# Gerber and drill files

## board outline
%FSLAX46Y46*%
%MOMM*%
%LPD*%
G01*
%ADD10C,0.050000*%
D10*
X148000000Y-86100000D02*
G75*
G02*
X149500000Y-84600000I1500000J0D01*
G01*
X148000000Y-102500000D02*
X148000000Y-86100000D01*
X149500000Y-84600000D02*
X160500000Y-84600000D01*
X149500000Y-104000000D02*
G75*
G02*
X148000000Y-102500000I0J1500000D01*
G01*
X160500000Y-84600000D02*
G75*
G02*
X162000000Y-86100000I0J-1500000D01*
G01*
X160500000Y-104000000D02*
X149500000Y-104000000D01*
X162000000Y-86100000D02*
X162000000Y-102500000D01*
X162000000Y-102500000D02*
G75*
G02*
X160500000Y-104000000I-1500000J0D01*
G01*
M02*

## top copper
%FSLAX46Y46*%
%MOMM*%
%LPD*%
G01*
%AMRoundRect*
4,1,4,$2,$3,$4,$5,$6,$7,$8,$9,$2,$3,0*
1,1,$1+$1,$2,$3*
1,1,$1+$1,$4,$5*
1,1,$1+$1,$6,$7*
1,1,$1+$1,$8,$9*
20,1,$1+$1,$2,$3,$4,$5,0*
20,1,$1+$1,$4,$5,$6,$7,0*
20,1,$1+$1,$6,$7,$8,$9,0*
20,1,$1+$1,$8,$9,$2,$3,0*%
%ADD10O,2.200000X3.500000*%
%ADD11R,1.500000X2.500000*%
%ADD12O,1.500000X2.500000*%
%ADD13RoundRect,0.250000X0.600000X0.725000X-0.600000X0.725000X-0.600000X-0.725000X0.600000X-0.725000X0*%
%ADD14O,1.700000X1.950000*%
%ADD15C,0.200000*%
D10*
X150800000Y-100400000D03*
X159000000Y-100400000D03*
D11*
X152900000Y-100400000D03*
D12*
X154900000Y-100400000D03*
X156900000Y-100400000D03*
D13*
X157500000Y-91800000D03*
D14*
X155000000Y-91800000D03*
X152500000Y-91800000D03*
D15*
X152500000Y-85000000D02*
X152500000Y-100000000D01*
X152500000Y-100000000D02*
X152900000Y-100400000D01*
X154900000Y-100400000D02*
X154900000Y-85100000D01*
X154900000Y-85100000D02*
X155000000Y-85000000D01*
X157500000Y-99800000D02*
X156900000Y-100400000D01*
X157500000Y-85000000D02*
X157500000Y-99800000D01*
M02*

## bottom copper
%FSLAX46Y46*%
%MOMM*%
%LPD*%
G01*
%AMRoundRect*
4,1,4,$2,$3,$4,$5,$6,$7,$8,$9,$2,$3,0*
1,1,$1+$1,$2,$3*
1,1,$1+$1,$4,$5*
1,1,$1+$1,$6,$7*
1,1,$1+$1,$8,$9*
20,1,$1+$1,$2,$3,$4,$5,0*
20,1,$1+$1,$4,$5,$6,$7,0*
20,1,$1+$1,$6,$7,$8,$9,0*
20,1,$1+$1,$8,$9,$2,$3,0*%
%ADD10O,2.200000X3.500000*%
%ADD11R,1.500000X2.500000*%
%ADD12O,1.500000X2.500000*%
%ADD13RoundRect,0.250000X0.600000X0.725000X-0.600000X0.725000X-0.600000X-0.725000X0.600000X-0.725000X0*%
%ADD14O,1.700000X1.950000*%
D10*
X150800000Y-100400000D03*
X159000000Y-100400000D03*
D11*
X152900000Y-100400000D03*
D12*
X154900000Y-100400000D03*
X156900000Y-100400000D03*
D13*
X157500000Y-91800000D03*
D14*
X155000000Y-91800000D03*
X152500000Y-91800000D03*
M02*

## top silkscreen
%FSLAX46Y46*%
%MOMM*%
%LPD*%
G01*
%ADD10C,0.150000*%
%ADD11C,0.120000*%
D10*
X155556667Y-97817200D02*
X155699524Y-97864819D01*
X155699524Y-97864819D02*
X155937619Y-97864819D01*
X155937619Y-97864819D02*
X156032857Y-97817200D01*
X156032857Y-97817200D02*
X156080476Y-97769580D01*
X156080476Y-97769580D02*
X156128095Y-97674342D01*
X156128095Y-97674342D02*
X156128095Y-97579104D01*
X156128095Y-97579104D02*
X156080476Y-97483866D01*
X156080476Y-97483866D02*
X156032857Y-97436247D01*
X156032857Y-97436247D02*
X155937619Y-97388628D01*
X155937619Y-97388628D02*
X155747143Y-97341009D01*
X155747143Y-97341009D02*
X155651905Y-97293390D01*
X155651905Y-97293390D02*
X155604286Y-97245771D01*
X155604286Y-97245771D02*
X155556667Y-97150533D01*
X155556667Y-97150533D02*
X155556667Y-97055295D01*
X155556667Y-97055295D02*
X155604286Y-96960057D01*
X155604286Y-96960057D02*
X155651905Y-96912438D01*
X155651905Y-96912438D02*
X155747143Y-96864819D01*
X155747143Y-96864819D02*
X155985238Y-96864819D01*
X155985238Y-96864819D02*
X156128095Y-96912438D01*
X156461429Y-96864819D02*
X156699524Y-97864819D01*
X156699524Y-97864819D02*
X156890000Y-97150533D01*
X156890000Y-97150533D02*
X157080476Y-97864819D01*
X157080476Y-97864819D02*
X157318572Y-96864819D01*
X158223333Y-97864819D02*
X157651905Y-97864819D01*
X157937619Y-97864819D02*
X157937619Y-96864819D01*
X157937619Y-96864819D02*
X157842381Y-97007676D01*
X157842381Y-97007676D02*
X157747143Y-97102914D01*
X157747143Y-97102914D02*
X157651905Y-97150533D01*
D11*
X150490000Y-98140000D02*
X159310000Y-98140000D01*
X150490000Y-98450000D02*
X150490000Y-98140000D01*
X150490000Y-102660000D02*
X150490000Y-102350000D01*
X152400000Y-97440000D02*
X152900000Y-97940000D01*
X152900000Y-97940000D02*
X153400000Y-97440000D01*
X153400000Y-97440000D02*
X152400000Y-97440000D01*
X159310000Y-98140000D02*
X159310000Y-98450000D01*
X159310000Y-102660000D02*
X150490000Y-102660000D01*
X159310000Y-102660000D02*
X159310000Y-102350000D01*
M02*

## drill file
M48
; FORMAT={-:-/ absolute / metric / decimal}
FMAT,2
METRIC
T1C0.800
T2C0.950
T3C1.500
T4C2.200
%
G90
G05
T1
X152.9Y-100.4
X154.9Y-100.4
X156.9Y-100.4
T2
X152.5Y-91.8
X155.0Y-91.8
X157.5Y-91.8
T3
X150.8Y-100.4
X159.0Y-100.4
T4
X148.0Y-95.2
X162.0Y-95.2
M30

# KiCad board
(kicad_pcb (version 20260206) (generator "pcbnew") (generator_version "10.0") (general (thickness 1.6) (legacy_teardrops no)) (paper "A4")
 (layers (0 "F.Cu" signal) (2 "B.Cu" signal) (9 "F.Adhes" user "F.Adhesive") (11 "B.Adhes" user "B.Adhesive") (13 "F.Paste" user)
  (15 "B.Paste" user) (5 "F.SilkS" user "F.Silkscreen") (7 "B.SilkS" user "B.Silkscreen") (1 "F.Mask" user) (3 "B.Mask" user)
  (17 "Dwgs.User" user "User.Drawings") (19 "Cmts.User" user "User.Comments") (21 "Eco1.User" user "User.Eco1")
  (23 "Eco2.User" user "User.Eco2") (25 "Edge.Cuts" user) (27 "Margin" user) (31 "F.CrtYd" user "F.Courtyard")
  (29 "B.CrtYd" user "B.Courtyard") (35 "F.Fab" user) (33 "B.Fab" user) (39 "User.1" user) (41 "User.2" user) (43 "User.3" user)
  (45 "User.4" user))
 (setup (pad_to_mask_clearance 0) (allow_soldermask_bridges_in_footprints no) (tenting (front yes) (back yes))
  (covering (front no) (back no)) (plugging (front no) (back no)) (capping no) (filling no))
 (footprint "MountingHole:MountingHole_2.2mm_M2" (layer "F.Cu") (at 162 95.2)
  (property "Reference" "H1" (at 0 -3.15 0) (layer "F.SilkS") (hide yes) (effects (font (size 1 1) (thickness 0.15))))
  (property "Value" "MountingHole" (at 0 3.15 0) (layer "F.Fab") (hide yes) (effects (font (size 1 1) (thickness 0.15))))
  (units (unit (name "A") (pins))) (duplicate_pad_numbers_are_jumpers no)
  (pad "" np_thru_hole circle (at 0 0) (size 2.2 2.2) (drill 2.2) (layers "*.Cu" "*.Mask")))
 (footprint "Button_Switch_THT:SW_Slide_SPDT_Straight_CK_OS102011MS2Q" (layer "F.Cu") (at 152.9 100.4)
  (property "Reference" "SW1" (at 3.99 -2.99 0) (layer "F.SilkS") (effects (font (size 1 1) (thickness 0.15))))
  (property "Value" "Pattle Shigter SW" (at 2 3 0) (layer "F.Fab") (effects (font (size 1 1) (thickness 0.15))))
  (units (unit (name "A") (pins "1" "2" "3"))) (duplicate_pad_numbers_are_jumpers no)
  (fp_line (start -2.41 -2.26) (end 6.41 -2.26) (stroke (width 0.12) (type solid)) (layer "F.SilkS"))
  (fp_line (start -2.41 -1.95) (end -2.41 -2.26) (stroke (width 0.12) (type solid)) (layer "F.SilkS"))
  (fp_line (start -2.41 2.26) (end -2.41 1.95) (stroke (width 0.12) (type solid)) (layer "F.SilkS"))
  (fp_line (start -0.5 -2.96) (end 0 -2.46) (stroke (width 0.12) (type solid)) (layer "F.SilkS"))
  (fp_line (start 0 -2.46) (end 0.5 -2.96) (stroke (width 0.12) (type solid)) (layer "F.SilkS"))
  (fp_line (start 0.5 -2.96) (end -0.5 -2.96) (stroke (width 0.12) (type solid)) (layer "F.SilkS"))
  (fp_line (start 6.41 -2.26) (end 6.41 -1.95) (stroke (width 0.12) (type solid)) (layer "F.SilkS"))
  (fp_line (start 6.41 2.26) (end -2.41 2.26) (stroke (width 0.12) (type solid)) (layer "F.SilkS"))
  (fp_line (start 6.41 2.26) (end 6.41 1.95) (stroke (width 0.12) (type solid)) (layer "F.SilkS"))
  (pad "" thru_hole oval (at -2.1 0) (size 2.2 3.5) (drill 1.5) (layers "*.Cu" "*.Mask") (remove_unused_layers no))
  (pad "" thru_hole oval (at 6.1 0) (size 2.2 3.5) (drill 1.5) (layers "*.Cu" "*.Mask") (remove_unused_layers no))
  (pad "1" thru_hole rect (at 0 0) (size 1.5 2.5) (drill 0.8) (layers "*.Cu" "*.Mask") (remove_unused_layers no) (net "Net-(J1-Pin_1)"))
  (pad "2" thru_hole oval (at 2 0) (size 1.5 2.5) (drill 0.8) (layers "*.Cu" "*.Mask") (remove_unused_layers no) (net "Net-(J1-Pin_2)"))
  (pad "3" thru_hole oval (at 4 0) (size 1.5 2.5) (drill 0.8) (layers "*.Cu" "*.Mask") (remove_unused_layers no) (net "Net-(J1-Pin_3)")))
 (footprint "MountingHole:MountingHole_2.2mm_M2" (layer "F.Cu") (at 148 95.2)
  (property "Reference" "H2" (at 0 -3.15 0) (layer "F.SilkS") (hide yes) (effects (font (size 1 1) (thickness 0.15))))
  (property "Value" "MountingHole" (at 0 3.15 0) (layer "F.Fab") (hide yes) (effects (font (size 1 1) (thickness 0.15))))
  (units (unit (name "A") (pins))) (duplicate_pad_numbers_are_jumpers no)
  (pad "" np_thru_hole circle (at 0 0) (size 2.2 2.2) (drill 2.2) (layers "*.Cu" "*.Mask")))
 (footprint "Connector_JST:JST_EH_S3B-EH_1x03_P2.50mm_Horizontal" (layer "B.Cu") (at 157.5 91.8 180)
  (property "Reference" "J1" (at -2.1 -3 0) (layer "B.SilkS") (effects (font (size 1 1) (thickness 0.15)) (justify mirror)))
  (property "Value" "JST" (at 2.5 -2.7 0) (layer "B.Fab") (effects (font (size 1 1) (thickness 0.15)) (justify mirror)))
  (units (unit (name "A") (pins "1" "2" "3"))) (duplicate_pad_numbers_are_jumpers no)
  (pad "1" thru_hole roundrect (at 0 0 180) (size 1.7 1.95) (drill 0.95) (layers "*.Cu" "*.Mask") (remove_unused_layers no)
   (roundrect_rratio 0.147059) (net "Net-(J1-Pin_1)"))
  (pad "2" thru_hole oval (at 2.5 0 180) (size 1.7 1.95) (drill 0.95) (layers "*.Cu" "*.Mask") (remove_unused_layers no)
   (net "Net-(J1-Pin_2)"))
  (pad "3" thru_hole oval (at 5 0 180) (size 1.7 1.95) (drill 0.95) (layers "*.Cu" "*.Mask") (remove_unused_layers no)
   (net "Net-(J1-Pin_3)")))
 (gr_arc (start 148 86.1) (mid 148.43934 85.03934) (end 149.5 84.6) (stroke (width 0.05) (type default)) (layer "Edge.Cuts"))
 (gr_line (start 148 102.5) (end 148 86.1) (stroke (width 0.05) (type default)) (layer "Edge.Cuts"))
 (gr_line (start 149.5 84.6) (end 160.5 84.6) (stroke (width 0.05) (type default)) (layer "Edge.Cuts"))
 (gr_arc (start 149.5 104) (mid 148.43934 103.56066) (end 148 102.5) (stroke (width 0.05) (type default)) (layer "Edge.Cuts"))
 (gr_arc (start 160.5 84.6) (mid 161.56066 85.03934) (end 162 86.1) (stroke (width 0.05) (type default)) (layer "Edge.Cuts"))
 (gr_line (start 160.5 104) (end 149.5 104) (stroke (width 0.05) (type default)) (layer "Edge.Cuts"))
 (gr_line (start 162 86.1) (end 162 102.5) (stroke (width 0.05) (type default)) (layer "Edge.Cuts"))
 (gr_arc (start 162 102.5) (mid 161.56066 103.56066) (end 160.5 104) (stroke (width 0.05) (type default)) (layer "Edge.Cuts"))
 (segment (start 152.5 85) (end 152.5 100) (width 0.2) (layer "F.Cu") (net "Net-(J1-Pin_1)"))
 (segment (start 152.5 100) (end 152.9 100.4) (width 0.2) (layer "F.Cu") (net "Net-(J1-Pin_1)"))
 (segment (start 154.9 100.4) (end 154.9 85.1) (width 0.2) (layer "F.Cu") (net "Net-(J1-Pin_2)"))
 (segment (start 154.9 85.1) (end 155 85) (width 0.2) (layer "F.Cu") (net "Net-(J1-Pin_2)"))
 (segment (start 157.5 99.8) (end 156.9 100.4) (width 0.2) (layer "F.Cu") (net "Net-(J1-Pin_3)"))
 (segment (start 157.5 85) (end 157.5 99.8) (width 0.2) (layer "F.Cu") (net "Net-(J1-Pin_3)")))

